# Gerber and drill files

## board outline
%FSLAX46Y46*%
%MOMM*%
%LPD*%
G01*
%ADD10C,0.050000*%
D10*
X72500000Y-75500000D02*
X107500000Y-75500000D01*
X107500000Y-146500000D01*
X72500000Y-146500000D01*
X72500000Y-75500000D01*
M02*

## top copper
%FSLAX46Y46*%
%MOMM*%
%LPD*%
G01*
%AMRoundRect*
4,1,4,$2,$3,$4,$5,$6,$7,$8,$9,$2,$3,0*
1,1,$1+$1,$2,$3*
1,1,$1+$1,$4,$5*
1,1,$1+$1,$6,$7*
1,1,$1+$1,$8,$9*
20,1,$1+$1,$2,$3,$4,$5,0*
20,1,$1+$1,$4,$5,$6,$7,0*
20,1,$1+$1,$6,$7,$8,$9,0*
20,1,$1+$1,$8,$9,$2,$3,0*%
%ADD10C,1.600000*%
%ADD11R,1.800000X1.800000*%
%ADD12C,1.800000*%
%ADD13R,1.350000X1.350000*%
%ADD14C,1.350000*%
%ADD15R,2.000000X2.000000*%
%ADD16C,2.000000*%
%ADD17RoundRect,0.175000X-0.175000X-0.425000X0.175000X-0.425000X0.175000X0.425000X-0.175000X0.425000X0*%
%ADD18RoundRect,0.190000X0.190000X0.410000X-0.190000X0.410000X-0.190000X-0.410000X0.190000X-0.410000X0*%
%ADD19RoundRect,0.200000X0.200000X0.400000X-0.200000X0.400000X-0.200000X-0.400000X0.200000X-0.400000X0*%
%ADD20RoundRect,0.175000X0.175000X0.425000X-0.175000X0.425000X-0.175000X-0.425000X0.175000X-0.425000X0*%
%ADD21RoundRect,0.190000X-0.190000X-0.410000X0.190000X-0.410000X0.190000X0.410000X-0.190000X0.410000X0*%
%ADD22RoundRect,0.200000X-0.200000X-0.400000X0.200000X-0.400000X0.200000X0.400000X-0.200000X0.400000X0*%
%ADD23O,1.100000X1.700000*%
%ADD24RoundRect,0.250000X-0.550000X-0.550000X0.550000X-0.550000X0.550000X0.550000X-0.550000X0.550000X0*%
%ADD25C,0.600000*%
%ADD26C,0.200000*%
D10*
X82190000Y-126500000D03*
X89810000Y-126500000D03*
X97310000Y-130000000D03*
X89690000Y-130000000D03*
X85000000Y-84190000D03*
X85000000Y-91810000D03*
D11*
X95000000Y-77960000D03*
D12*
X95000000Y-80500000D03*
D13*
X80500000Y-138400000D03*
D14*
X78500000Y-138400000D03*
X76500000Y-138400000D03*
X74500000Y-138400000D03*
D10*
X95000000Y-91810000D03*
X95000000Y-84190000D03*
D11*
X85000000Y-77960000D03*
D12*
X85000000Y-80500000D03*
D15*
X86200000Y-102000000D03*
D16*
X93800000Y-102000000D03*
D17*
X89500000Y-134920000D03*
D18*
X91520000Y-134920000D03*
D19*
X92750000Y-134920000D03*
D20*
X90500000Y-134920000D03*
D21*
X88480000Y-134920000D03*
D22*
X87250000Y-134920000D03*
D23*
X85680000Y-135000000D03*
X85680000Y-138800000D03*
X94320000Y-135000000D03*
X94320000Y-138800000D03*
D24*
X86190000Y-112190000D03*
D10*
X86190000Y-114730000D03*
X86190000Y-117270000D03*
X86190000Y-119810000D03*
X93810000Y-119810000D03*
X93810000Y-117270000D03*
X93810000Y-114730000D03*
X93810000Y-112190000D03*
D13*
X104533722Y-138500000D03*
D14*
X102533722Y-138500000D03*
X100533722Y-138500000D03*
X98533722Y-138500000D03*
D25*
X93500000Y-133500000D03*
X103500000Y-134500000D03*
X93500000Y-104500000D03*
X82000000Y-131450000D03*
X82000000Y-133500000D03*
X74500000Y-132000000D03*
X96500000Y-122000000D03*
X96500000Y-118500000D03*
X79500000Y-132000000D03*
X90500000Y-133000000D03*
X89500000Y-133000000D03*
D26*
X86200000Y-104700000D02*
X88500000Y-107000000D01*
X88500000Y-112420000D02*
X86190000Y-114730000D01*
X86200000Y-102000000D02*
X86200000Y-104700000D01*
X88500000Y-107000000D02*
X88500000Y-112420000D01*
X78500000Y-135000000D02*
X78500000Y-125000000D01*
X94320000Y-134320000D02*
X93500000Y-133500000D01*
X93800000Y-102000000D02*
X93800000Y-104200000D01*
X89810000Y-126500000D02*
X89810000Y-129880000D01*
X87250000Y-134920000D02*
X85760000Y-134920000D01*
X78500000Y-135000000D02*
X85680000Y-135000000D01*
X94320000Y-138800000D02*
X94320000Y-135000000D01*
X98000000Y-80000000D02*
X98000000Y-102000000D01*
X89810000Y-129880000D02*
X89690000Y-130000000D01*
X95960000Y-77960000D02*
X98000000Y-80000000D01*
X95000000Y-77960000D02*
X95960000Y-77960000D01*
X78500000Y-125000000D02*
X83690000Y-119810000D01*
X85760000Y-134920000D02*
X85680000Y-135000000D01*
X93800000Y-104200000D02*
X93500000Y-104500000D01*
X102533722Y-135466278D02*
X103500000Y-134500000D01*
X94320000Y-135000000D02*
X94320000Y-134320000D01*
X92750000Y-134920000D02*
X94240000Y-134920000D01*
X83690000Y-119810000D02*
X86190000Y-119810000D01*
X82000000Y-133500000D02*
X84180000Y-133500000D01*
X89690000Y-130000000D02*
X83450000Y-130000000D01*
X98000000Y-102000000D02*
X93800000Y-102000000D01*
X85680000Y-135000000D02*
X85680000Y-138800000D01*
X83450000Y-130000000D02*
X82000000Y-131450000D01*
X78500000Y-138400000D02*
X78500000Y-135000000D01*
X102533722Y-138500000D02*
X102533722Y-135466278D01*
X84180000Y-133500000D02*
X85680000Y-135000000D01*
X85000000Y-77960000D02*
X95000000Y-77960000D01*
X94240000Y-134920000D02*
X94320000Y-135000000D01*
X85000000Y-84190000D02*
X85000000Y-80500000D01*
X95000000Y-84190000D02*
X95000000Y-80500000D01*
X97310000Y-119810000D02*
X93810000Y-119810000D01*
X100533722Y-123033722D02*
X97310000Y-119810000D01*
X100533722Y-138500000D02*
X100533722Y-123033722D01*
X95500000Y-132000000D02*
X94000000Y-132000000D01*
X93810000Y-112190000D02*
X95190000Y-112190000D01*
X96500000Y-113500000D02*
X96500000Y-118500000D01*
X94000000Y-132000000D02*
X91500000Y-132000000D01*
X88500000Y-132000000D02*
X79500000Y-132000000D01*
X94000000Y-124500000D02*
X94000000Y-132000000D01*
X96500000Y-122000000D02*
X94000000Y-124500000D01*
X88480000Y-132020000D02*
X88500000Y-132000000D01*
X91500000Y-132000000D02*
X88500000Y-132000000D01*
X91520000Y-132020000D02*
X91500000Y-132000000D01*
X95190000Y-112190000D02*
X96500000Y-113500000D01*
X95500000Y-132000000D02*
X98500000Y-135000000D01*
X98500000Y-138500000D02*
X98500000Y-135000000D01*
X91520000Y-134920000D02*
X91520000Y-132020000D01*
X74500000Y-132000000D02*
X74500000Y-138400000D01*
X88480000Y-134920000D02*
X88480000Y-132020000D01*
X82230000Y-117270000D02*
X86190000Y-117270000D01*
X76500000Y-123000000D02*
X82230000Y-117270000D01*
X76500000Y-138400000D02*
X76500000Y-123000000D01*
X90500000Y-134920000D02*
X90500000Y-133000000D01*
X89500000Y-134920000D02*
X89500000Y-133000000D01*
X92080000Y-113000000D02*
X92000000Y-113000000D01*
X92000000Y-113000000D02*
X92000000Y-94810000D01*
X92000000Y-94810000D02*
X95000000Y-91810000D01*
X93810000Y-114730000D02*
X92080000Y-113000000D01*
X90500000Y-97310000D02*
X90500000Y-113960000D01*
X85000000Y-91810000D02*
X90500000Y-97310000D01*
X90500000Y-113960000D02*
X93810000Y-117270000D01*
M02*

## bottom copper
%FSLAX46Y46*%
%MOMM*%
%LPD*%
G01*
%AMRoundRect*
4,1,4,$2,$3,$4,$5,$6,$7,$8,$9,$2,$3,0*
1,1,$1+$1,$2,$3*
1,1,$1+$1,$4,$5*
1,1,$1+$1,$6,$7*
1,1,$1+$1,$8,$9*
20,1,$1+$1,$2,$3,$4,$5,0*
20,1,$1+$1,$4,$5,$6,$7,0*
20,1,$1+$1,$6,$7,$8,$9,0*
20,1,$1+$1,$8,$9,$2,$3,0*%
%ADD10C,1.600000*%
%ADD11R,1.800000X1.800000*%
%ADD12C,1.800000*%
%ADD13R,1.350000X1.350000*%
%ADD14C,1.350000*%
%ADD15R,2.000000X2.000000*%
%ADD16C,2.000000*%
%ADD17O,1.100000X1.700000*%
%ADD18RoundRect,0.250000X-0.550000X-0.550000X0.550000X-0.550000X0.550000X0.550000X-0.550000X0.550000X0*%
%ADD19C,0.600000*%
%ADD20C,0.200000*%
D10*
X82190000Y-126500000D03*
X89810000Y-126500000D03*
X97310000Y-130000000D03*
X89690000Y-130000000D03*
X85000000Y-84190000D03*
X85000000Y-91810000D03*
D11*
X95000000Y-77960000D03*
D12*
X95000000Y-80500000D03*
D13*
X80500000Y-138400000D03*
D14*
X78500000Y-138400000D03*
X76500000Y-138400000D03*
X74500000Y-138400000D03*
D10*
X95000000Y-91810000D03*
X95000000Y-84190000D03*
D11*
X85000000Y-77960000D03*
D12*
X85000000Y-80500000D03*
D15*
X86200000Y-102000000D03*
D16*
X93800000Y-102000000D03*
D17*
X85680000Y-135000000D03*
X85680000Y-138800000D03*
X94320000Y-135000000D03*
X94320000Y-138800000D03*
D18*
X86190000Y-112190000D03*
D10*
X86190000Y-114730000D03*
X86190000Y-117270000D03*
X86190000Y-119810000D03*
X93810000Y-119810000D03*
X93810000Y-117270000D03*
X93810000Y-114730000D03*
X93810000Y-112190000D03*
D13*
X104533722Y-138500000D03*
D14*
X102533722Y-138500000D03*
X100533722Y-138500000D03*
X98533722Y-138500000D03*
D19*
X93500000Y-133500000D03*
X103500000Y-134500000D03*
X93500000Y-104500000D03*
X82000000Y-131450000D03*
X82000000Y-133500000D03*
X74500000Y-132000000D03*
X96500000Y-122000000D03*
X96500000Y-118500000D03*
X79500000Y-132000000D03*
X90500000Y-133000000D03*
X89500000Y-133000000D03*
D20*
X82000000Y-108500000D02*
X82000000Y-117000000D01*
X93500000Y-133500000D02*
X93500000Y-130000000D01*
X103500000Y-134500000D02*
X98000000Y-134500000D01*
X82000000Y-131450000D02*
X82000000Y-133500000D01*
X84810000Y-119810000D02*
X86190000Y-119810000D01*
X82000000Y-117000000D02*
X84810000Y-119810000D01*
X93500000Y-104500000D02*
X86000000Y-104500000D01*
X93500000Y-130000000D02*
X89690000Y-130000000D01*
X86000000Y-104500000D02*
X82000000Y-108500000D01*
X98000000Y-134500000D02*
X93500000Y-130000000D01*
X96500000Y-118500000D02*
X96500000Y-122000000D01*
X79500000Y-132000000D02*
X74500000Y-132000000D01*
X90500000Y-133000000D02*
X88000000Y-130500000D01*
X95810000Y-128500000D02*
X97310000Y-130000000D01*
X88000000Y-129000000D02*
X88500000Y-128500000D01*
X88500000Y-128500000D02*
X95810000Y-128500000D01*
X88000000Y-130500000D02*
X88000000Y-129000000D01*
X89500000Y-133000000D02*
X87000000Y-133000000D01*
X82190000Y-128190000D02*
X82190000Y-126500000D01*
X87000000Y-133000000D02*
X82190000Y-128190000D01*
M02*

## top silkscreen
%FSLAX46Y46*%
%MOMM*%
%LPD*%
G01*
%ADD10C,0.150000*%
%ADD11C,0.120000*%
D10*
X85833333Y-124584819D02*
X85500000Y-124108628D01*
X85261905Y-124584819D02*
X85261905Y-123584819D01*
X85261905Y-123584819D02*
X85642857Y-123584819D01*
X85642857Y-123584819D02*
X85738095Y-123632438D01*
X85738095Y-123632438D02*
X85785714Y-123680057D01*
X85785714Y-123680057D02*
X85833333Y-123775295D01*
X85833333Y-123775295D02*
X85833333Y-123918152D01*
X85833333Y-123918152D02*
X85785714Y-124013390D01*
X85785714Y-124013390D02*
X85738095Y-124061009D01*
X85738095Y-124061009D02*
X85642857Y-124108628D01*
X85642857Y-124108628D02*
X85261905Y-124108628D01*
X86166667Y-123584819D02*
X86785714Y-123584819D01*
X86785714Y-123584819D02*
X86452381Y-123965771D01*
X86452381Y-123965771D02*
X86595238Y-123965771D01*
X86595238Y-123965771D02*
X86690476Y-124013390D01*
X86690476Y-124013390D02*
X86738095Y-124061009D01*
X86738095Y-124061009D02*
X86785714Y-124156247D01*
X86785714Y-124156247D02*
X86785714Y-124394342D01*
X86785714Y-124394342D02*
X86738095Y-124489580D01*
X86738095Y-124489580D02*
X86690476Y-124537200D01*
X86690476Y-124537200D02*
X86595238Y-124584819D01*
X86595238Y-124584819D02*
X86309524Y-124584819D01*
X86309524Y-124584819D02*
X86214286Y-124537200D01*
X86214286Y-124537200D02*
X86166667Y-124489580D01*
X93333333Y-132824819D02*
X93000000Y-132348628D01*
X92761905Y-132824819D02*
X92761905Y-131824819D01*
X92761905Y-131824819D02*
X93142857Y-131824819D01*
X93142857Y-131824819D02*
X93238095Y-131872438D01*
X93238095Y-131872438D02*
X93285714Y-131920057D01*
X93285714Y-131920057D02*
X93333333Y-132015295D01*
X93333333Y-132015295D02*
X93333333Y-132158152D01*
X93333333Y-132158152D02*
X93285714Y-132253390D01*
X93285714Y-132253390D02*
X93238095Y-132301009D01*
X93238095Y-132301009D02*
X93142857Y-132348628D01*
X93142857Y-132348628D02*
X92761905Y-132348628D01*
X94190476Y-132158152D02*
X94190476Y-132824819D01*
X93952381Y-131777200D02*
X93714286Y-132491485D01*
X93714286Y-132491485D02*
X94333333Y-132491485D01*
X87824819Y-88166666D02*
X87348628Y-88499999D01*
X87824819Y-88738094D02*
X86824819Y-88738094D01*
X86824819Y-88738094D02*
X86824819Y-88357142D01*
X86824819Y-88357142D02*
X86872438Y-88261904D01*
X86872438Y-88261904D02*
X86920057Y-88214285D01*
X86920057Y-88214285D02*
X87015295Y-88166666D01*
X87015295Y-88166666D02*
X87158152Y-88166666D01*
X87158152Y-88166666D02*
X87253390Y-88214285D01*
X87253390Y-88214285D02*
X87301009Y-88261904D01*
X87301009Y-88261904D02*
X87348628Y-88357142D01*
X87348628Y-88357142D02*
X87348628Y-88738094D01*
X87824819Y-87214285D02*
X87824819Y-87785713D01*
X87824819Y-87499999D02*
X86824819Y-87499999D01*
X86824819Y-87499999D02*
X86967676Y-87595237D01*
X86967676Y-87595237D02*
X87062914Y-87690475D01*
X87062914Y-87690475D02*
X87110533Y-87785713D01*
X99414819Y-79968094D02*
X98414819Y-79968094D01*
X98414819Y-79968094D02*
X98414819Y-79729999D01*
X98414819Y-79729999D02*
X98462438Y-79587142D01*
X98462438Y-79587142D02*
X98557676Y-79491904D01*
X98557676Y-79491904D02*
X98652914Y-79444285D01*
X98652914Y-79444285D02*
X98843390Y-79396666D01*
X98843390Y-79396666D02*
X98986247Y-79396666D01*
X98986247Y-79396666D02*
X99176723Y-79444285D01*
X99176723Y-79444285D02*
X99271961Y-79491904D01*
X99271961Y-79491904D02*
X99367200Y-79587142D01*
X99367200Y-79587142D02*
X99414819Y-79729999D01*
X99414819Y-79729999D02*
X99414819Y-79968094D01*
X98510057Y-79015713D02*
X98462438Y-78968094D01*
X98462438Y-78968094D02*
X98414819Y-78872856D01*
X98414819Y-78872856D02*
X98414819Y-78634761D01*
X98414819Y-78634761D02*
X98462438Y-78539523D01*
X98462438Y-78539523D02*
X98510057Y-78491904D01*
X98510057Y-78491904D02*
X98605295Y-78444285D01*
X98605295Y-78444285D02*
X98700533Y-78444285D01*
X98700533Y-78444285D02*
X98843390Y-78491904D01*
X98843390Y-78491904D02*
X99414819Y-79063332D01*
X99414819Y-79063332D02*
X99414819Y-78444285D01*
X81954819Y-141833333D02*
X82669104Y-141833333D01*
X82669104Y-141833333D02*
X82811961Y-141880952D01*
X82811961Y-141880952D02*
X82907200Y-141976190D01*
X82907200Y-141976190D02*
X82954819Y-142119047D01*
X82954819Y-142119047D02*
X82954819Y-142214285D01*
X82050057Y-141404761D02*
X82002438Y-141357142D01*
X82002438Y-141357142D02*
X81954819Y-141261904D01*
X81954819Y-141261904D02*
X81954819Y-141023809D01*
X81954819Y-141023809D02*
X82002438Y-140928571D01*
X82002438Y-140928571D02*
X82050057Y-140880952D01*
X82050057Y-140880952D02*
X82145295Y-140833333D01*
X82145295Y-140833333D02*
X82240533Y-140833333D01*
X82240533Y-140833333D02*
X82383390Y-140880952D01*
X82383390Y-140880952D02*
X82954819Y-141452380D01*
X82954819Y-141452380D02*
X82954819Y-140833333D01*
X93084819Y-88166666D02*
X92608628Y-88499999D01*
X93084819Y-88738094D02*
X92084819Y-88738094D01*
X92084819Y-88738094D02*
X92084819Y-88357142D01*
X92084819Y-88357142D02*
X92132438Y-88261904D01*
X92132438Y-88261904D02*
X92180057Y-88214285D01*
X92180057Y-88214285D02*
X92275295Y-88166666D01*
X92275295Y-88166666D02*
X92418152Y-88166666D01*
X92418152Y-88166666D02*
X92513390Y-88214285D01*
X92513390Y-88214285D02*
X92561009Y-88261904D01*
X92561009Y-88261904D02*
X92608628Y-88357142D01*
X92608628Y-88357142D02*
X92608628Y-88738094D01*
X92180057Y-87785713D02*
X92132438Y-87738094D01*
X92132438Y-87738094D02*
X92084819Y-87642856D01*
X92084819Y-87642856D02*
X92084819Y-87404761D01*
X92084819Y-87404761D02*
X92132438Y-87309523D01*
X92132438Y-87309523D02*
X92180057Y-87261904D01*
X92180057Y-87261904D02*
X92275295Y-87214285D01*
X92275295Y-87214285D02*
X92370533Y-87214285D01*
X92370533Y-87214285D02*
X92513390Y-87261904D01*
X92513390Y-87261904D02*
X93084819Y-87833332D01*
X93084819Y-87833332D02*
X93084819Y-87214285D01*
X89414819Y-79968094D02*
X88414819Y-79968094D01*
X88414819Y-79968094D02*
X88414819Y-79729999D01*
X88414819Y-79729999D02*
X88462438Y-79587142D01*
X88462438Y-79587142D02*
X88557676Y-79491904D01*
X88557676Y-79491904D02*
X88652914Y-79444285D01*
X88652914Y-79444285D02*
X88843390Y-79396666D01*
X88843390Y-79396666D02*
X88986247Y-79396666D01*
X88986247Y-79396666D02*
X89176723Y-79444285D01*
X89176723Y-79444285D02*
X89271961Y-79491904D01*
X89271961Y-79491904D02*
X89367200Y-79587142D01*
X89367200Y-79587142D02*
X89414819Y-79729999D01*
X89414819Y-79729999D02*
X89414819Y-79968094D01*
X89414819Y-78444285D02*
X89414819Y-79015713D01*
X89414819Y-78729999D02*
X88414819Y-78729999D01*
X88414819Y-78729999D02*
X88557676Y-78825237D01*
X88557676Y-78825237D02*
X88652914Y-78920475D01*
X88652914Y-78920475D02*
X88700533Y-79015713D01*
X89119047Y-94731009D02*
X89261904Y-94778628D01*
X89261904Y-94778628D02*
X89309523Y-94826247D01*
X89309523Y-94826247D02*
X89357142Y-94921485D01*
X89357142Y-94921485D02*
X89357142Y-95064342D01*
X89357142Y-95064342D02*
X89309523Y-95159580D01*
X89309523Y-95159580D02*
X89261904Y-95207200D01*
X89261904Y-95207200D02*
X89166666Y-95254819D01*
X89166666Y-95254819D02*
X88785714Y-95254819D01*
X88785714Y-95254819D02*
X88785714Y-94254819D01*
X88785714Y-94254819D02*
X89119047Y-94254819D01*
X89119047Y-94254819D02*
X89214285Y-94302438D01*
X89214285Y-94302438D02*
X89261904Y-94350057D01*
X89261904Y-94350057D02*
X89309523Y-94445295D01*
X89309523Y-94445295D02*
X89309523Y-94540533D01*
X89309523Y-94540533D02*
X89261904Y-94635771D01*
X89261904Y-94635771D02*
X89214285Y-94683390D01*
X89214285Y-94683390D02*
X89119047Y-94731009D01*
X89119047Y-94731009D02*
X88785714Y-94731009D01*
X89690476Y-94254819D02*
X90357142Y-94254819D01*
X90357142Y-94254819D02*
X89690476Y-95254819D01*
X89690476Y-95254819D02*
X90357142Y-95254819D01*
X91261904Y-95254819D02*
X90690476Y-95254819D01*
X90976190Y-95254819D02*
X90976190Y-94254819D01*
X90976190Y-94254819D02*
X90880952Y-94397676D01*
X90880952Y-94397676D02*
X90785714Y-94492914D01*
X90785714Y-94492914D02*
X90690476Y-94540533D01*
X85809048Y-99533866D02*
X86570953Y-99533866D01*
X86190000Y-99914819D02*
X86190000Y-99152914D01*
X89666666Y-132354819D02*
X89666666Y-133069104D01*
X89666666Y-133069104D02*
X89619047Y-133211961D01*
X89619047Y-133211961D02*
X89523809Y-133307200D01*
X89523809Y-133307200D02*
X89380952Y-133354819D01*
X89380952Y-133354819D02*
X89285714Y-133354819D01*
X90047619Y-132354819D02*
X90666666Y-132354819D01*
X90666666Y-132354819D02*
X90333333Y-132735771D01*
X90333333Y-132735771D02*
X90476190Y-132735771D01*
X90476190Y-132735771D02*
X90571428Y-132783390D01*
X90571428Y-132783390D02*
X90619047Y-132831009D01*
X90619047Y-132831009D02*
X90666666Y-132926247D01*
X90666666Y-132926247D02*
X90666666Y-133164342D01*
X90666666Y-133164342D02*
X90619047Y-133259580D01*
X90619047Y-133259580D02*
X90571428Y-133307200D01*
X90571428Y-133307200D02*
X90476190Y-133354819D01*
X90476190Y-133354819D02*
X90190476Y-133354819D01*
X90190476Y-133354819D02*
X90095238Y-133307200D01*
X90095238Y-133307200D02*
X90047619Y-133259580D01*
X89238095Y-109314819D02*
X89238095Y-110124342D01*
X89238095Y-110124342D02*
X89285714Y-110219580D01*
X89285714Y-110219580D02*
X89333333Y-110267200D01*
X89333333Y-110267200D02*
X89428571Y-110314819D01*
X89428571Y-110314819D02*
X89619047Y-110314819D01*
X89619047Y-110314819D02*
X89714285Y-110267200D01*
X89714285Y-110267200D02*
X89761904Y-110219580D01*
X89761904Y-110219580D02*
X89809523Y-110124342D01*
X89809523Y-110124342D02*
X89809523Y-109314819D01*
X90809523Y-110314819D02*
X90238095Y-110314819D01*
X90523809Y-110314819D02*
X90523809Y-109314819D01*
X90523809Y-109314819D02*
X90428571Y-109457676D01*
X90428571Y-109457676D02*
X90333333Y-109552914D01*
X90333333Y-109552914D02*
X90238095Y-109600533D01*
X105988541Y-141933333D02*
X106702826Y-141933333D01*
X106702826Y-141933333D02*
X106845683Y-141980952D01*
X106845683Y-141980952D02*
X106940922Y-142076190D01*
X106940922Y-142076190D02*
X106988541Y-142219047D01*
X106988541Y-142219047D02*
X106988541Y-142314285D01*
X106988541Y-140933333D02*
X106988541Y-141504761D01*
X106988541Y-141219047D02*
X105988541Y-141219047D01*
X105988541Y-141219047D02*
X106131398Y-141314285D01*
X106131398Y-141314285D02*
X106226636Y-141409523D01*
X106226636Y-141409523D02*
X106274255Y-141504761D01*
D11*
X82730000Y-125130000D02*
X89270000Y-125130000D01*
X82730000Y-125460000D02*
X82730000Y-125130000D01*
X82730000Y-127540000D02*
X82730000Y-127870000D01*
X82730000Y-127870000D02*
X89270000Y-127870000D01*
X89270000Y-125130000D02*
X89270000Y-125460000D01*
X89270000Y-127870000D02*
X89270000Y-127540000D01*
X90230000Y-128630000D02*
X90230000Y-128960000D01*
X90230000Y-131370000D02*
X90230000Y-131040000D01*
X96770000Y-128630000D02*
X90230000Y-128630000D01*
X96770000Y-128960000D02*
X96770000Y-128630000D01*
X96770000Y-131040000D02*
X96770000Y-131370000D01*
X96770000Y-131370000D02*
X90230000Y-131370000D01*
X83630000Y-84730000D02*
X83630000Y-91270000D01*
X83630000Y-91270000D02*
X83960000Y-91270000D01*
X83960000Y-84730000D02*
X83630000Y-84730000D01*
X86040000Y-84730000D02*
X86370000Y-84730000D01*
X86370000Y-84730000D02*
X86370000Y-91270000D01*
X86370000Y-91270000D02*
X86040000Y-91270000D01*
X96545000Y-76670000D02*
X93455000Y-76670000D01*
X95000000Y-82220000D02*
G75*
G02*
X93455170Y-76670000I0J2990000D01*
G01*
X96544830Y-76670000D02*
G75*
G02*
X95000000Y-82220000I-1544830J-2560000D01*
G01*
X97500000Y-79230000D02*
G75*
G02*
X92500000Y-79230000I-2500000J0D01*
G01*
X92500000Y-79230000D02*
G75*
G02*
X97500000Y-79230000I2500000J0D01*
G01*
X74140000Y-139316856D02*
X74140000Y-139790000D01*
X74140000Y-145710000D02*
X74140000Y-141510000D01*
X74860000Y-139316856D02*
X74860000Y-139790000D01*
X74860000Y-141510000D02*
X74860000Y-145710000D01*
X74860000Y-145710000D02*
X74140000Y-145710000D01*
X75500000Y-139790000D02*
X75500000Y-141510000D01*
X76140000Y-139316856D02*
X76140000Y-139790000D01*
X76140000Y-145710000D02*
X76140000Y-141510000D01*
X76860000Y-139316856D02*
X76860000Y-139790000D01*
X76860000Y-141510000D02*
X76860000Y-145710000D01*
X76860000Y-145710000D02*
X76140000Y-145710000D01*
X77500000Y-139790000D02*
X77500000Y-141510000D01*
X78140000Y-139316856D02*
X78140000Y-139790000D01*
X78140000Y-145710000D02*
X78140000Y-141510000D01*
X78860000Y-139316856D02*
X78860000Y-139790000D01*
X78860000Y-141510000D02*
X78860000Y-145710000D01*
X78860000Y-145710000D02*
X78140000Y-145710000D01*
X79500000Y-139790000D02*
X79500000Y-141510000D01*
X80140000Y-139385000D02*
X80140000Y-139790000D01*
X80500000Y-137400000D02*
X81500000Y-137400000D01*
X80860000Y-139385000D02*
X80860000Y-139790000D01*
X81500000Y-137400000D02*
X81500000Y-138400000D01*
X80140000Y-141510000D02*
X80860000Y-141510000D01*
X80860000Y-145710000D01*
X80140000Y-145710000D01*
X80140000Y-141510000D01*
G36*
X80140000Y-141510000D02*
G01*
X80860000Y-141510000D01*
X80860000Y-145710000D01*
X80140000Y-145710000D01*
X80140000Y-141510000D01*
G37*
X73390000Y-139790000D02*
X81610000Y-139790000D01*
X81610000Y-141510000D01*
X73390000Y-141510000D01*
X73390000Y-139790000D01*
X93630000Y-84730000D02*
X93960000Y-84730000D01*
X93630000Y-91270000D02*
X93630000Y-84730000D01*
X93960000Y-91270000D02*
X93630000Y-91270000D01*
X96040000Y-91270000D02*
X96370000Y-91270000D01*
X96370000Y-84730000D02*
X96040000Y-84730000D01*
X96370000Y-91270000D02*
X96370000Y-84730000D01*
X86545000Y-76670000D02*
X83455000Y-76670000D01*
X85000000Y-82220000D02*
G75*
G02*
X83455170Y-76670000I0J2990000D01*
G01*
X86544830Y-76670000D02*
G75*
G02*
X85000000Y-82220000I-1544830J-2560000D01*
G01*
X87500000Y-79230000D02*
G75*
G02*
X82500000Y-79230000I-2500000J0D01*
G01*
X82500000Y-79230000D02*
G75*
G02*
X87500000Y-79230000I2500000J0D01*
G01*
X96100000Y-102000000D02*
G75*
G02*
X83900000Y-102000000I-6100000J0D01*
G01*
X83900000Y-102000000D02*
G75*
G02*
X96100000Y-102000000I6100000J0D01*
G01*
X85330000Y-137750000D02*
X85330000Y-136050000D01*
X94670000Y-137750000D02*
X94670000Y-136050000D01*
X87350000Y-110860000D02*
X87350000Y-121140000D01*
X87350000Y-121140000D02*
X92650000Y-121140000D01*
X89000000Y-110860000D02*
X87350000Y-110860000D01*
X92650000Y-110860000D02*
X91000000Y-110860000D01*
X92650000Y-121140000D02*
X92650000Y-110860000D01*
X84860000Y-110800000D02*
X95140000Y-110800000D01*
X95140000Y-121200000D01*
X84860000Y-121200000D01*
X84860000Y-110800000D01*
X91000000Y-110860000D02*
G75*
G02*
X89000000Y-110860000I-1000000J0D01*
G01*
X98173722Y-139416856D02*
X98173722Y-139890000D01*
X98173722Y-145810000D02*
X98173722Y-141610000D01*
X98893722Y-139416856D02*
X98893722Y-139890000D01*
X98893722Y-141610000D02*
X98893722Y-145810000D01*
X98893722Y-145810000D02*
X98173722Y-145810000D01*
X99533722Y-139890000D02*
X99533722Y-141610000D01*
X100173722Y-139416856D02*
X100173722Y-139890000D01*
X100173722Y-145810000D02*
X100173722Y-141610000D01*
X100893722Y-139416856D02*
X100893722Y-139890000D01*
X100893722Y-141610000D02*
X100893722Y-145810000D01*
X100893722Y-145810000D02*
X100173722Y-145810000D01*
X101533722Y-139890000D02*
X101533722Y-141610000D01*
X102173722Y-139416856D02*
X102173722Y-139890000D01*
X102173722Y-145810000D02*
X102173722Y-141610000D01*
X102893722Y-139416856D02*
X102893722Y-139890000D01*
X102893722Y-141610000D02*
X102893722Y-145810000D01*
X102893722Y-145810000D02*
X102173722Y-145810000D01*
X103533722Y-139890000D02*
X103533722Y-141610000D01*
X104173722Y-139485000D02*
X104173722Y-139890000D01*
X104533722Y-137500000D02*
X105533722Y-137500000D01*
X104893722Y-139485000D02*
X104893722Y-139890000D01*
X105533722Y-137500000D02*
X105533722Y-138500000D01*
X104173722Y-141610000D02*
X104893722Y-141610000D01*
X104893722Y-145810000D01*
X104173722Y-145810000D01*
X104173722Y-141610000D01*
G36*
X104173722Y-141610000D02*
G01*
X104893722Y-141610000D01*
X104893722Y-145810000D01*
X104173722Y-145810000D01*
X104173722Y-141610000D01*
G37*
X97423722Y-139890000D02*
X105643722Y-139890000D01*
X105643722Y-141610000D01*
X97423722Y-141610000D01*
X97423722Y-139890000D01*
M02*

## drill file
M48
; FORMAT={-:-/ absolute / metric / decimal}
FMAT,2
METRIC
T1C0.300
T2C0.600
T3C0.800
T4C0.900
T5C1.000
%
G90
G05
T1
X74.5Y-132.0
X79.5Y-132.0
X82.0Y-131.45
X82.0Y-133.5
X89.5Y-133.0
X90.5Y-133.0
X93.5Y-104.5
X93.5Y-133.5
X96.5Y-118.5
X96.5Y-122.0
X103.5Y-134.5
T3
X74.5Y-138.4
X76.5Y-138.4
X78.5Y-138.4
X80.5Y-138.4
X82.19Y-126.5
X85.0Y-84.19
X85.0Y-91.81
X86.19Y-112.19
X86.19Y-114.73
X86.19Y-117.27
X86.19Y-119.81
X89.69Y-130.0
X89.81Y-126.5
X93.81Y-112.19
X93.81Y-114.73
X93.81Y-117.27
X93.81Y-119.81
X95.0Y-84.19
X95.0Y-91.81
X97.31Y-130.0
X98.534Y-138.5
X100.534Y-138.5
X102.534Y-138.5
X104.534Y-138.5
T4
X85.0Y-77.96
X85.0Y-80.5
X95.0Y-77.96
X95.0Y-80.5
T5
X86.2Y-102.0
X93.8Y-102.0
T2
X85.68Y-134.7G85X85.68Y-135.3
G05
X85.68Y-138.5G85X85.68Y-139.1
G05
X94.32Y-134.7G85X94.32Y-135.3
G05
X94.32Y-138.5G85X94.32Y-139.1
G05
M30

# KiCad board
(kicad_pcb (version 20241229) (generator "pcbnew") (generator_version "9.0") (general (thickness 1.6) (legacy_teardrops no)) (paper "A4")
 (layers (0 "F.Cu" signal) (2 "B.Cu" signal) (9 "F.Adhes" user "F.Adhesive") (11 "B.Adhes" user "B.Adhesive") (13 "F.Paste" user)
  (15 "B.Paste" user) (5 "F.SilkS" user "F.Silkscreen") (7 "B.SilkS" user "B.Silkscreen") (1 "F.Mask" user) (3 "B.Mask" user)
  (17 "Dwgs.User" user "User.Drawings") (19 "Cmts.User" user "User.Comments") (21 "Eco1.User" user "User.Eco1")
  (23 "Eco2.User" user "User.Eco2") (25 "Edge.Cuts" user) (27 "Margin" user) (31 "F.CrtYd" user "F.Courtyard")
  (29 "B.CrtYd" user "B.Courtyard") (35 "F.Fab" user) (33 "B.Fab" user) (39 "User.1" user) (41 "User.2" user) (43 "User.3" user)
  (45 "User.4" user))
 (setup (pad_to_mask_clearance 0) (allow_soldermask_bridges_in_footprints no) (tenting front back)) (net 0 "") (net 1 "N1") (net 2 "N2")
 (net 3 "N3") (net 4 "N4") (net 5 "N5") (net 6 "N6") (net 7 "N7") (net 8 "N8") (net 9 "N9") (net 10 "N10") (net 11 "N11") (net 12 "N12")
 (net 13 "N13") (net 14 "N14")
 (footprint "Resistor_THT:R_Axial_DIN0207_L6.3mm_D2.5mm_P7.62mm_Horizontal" (layer "F.Cu") (at 82.19 126.5)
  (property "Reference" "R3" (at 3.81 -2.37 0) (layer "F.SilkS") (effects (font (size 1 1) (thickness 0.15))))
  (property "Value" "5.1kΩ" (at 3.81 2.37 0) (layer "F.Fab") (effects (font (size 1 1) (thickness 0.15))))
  (fp_line (start 0.54 -1.37) (end 7.08 -1.37) (stroke (width 0.12) (type solid)) (layer "F.SilkS"))
  (fp_line (start 0.54 -1.04) (end 0.54 -1.37) (stroke (width 0.12) (type solid)) (layer "F.SilkS"))
  (fp_line (start 0.54 1.04) (end 0.54 1.37) (stroke (width 0.12) (type solid)) (layer "F.SilkS"))
  (fp_line (start 0.54 1.37) (end 7.08 1.37) (stroke (width 0.12) (type solid)) (layer "F.SilkS"))
  (fp_line (start 7.08 -1.37) (end 7.08 -1.04) (stroke (width 0.12) (type solid)) (layer "F.SilkS"))
  (fp_line (start 7.08 1.37) (end 7.08 1.04) (stroke (width 0.12) (type solid)) (layer "F.SilkS"))
  (pad "1" thru_hole circle (at 0 0) (size 1.6 1.6) (drill 0.8) (layers "*.Cu" "*.Mask") (remove_unused_layers no) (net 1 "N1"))
  (pad "2" thru_hole circle (at 7.62 0) (size 1.6 1.6) (drill 0.8) (layers "*.Cu" "*.Mask") (remove_unused_layers no) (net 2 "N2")))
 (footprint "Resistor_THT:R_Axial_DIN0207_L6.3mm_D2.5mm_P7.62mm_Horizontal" (layer "F.Cu") (at 97.31 130 180)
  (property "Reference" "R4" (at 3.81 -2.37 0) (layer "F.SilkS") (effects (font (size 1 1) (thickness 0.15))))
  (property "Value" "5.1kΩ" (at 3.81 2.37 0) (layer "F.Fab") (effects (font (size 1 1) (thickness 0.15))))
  (fp_line (start 7.08 1.37) (end 7.08 1.04) (stroke (width 0.12) (type solid)) (layer "F.SilkS"))
  (fp_line (start 7.08 -1.37) (end 7.08 -1.04) (stroke (width 0.12) (type solid)) (layer "F.SilkS"))
  (fp_line (start 0.54 1.37) (end 7.08 1.37) (stroke (width 0.12) (type solid)) (layer "F.SilkS"))
  (fp_line (start 0.54 1.04) (end 0.54 1.37) (stroke (width 0.12) (type solid)) (layer "F.SilkS"))
  (fp_line (start 0.54 -1.04) (end 0.54 -1.37) (stroke (width 0.12) (type solid)) (layer "F.SilkS"))
  (fp_line (start 0.54 -1.37) (end 7.08 -1.37) (stroke (width 0.12) (type solid)) (layer "F.SilkS"))
  (pad "1" thru_hole circle (at 0 0 180) (size 1.6 1.6) (drill 0.8) (layers "*.Cu" "*.Mask") (remove_unused_layers no) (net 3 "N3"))
  (pad "2" thru_hole circle (at 7.62 0 180) (size 1.6 1.6) (drill 0.8) (layers "*.Cu" "*.Mask") (remove_unused_layers no) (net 2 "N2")))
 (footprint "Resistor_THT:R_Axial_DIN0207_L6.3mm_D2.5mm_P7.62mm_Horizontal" (layer "F.Cu") (at 85 84.19 -90)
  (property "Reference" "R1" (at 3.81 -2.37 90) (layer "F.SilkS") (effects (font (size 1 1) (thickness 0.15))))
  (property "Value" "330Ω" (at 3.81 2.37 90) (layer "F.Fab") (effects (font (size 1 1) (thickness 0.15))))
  (fp_line (start 0.54 1.37) (end 7.08 1.37) (stroke (width 0.12) (type solid)) (layer "F.SilkS"))
  (fp_line (start 7.08 1.37) (end 7.08 1.04) (stroke (width 0.12) (type solid)) (layer "F.SilkS"))
  (fp_line (start 0.54 1.04) (end 0.54 1.37) (stroke (width 0.12) (type solid)) (layer "F.SilkS"))
  (fp_line (start 0.54 -1.04) (end 0.54 -1.37) (stroke (width 0.12) (type solid)) (layer "F.SilkS"))
  (fp_line (start 0.54 -1.37) (end 7.08 -1.37) (stroke (width 0.12) (type solid)) (layer "F.SilkS"))
  (fp_line (start 7.08 -1.37) (end 7.08 -1.04) (stroke (width 0.12) (type solid)) (layer "F.SilkS"))
  (pad "1" thru_hole circle (at 0 0 270) (size 1.6 1.6) (drill 0.8) (layers "*.Cu" "*.Mask") (remove_unused_layers no) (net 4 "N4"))
  (pad "2" thru_hole circle (at 7.62 0 270) (size 1.6 1.6) (drill 0.8) (layers "*.Cu" "*.Mask") (remove_unused_layers no) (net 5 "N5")))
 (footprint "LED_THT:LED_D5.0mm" (layer "F.Cu") (at 95 77.96 -90)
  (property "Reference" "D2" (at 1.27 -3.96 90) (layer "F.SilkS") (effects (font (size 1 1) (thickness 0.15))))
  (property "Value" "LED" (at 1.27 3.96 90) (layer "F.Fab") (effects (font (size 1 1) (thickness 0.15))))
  (fp_line (start -1.29 -1.545) (end -1.29 1.545) (stroke (width 0.12) (type solid)) (layer "F.SilkS"))
  (fp_arc (start 4.26 0) (mid 2.071779 2.880495) (end -1.29 1.54483) (stroke (width 0.12) (type solid)) (layer "F.SilkS"))
  (fp_arc (start -1.29 -1.54483) (mid 2.071779 -2.880495) (end 4.26 0) (stroke (width 0.12) (type solid)) (layer "F.SilkS"))
  (fp_circle (center 1.27 0) (end 3.77 0) (stroke (width 0.12) (type solid)) (fill no) (layer "F.SilkS"))
  (pad "1" thru_hole rect (at 0 0 270) (size 1.8 1.8) (drill 0.9) (layers "*.Cu" "*.Mask") (remove_unused_layers no) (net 2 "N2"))
  (pad "2" thru_hole circle (at 2.54 0 270) (size 1.8 1.8) (drill 0.9) (layers "*.Cu" "*.Mask") (remove_unused_layers no) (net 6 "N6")))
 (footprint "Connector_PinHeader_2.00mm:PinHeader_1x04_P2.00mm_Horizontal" (layer "F.Cu") (at 80.5 138.4 -90)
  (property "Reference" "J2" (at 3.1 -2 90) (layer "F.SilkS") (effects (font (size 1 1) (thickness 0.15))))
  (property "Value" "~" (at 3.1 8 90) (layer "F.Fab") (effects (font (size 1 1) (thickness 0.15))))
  (fp_line (start 0.916856 6.36) (end 1.39 6.36) (stroke (width 0.12) (type solid)) (layer "F.SilkS"))
  (fp_line (start 7.31 6.36) (end 3.11 6.36) (stroke (width 0.12) (type solid)) (layer "F.SilkS"))
  (fp_line (start 0.916856 5.64) (end 1.39 5.64) (stroke (width 0.12) (type solid)) (layer "F.SilkS"))
  (fp_line (start 3.11 5.64) (end 7.31 5.64) (stroke (width 0.12) (type solid)) (layer "F.SilkS"))
  (fp_line (start 7.31 5.64) (end 7.31 6.36) (stroke (width 0.12) (type solid)) (layer "F.SilkS"))
  (fp_line (start 1.39 5) (end 3.11 5) (stroke (width 0.12) (type solid)) (layer "F.SilkS"))
  (fp_line (start 0.916856 4.36) (end 1.39 4.36) (stroke (width 0.12) (type solid)) (layer "F.SilkS"))
  (fp_line (start 7.31 4.36) (end 3.11 4.36) (stroke (width 0.12) (type solid)) (layer "F.SilkS"))
  (fp_line (start 0.916856 3.64) (end 1.39 3.64) (stroke (width 0.12) (type solid)) (layer "F.SilkS"))
  (fp_line (start 3.11 3.64) (end 7.31 3.64) (stroke (width 0.12) (type solid)) (layer "F.SilkS"))
  (fp_line (start 7.31 3.64) (end 7.31 4.36) (stroke (width 0.12) (type solid)) (layer "F.SilkS"))
  (fp_line (start 1.39 3) (end 3.11 3) (stroke (width 0.12) (type solid)) (layer "F.SilkS"))
  (fp_line (start 0.916856 2.36) (end 1.39 2.36) (stroke (width 0.12) (type solid)) (layer "F.SilkS"))
  (fp_line (start 7.31 2.36) (end 3.11 2.36) (stroke (width 0.12) (type solid)) (layer "F.SilkS"))
  (fp_line (start 0.916856 1.64) (end 1.39 1.64) (stroke (width 0.12) (type solid)) (layer "F.SilkS"))
  (fp_line (start 3.11 1.64) (end 7.31 1.64) (stroke (width 0.12) (type solid)) (layer "F.SilkS"))
  (fp_line (start 7.31 1.64) (end 7.31 2.36) (stroke (width 0.12) (type solid)) (layer "F.SilkS"))
  (fp_line (start 1.39 1) (end 3.11 1) (stroke (width 0.12) (type solid)) (layer "F.SilkS"))
  (fp_line (start 0.985 0.36) (end 1.39 0.36) (stroke (width 0.12) (type solid)) (layer "F.SilkS"))
  (fp_line (start -1 0) (end -1 -1) (stroke (width 0.12) (type solid)) (layer "F.SilkS"))
  (fp_line (start 0.985 -0.36) (end 1.39 -0.36) (stroke (width 0.12) (type solid)) (layer "F.SilkS"))
  (fp_line (start -1 -1) (end 0 -1) (stroke (width 0.12) (type solid)) (layer "F.SilkS"))
  (fp_rect (start 3.11 -0.36) (end 7.31 0.36) (stroke (width 0.12) (type solid)) (fill yes) (layer "F.SilkS"))
  (fp_rect (start 1.39 -1.11) (end 3.11 7.11) (stroke (width 0.12) (type solid)) (fill no) (layer "F.SilkS"))
  (pad "1" thru_hole rect (at 0 0 270) (size 1.35 1.35) (drill 0.8) (layers "*.Cu" "*.Mask") (remove_unused_layers no) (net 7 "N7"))
  (pad "2" thru_hole circle (at 0 2 270) (size 1.35 1.35) (drill 0.8) (layers "*.Cu" "*.Mask") (remove_unused_layers no) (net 2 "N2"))
  (pad "3" thru_hole circle (at 0 4 270) (size 1.35 1.35) (drill 0.8) (layers "*.Cu" "*.Mask") (remove_unused_layers no) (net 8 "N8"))
  (pad "4" thru_hole circle (at 0 6 270) (size 1.35 1.35) (drill 0.8) (layers "*.Cu" "*.Mask") (remove_unused_layers no) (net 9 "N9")))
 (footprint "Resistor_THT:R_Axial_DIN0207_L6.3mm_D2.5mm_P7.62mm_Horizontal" (layer "F.Cu") (at 95 91.81 90)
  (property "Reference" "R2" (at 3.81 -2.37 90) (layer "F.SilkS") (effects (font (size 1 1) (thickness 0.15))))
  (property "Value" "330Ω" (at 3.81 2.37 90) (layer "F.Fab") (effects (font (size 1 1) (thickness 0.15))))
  (fp_line (start 7.08 -1.37) (end 7.08 -1.04) (stroke (width 0.12) (type solid)) (layer "F.SilkS"))
  (fp_line (start 0.54 -1.37) (end 7.08 -1.37) (stroke (width 0.12) (type solid)) (layer "F.SilkS"))
  (fp_line (start 0.54 -1.04) (end 0.54 -1.37) (stroke (width 0.12) (type solid)) (layer "F.SilkS"))
  (fp_line (start 0.54 1.04) (end 0.54 1.37) (stroke (width 0.12) (type solid)) (layer "F.SilkS"))
  (fp_line (start 7.08 1.37) (end 7.08 1.04) (stroke (width 0.12) (type solid)) (layer "F.SilkS"))
  (fp_line (start 0.54 1.37) (end 7.08 1.37) (stroke (width 0.12) (type solid)) (layer "F.SilkS"))
  (pad "1" thru_hole circle (at 0 0 90) (size 1.6 1.6) (drill 0.8) (layers "*.Cu" "*.Mask") (remove_unused_layers no) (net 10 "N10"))
  (pad "2" thru_hole circle (at 7.62 0 90) (size 1.6 1.6) (drill 0.8) (layers "*.Cu" "*.Mask") (remove_unused_layers no) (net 6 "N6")))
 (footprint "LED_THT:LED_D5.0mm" (layer "F.Cu") (at 85 77.96 -90)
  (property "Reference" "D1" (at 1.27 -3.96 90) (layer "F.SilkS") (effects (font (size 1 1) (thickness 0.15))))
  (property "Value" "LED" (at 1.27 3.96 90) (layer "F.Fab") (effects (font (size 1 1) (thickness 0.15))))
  (fp_line (start -1.29 -1.545) (end -1.29 1.545) (stroke (width 0.12) (type solid)) (layer "F.SilkS"))
  (fp_arc (start 4.26 0) (mid 2.071779 2.880495) (end -1.29 1.54483) (stroke (width 0.12) (type solid)) (layer "F.SilkS"))
  (fp_arc (start -1.29 -1.54483) (mid 2.071779 -2.880495) (end 4.26 0) (stroke (width 0.12) (type solid)) (layer "F.SilkS"))
  (fp_circle (center 1.27 0) (end 3.77 0) (stroke (width 0.12) (type solid)) (fill no) (layer "F.SilkS"))
  (pad "1" thru_hole rect (at 0 0 270) (size 1.8 1.8) (drill 0.9) (layers "*.Cu" "*.Mask") (remove_unused_layers no) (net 2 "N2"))
  (pad "2" thru_hole circle (at 2.54 0 270) (size 1.8 1.8) (drill 0.9) (layers "*.Cu" "*.Mask") (remove_unused_layers no) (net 4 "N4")))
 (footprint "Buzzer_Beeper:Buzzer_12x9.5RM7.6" (layer "F.Cu") (at 86.2 102)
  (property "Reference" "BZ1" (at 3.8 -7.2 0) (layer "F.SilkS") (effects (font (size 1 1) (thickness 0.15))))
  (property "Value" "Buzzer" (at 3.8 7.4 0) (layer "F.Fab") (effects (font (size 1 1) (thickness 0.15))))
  (fp_circle (center 3.8 0) (end 9.9 0) (stroke (width 0.12) (type solid)) (fill no) (layer "F.SilkS"))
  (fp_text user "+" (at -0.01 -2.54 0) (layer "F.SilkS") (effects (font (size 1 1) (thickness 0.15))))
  (pad "1" thru_hole rect (at 0 0) (size 2 2) (drill 1) (layers "*.Cu" "*.Mask") (remove_unused_layers no) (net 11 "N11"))
  (pad "2" thru_hole circle (at 7.6 0) (size 2 2) (drill 1) (layers "*.Cu" "*.Mask") (remove_unused_layers no) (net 2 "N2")))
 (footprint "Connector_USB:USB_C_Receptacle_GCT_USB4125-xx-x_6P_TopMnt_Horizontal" (layer "F.Cu") (at 90 138)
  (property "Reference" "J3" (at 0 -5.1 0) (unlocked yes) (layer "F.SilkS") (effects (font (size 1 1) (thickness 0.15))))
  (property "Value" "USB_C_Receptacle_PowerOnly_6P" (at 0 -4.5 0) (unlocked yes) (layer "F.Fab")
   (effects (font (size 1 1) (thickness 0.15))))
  (fp_line (start -4.67 -0.25) (end -4.67 -1.95) (stroke (width 0.12) (type solid)) (layer "F.SilkS"))
  (fp_line (start 4.67 -0.25) (end 4.67 -1.95) (stroke (width 0.12) (type solid)) (layer "F.SilkS"))
  (pad "A5" smd roundrect (at -0.5 -3.08) (size 0.7 1.2) (layers "F.Cu" "F.Mask" "F.Paste") (roundrect_rratio 0.25) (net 1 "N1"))
  (pad "A9" smd roundrect (at 1.52 -3.08 180) (size 0.76 1.2) (layers "F.Cu" "F.Mask" "F.Paste") (roundrect_rratio 0.25) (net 9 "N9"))
  (pad "A12" smd roundrect (at 2.75 -3.08 180) (size 0.8 1.2) (layers "F.Cu" "F.Mask" "F.Paste") (roundrect_rratio 0.25) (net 2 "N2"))
  (pad "B5" smd roundrect (at 0.5 -3.08 180) (size 0.7 1.2) (layers "F.Cu" "F.Mask" "F.Paste") (roundrect_rratio 0.25) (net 3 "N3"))
  (pad "B9" smd roundrect (at -1.52 -3.08) (size 0.76 1.2) (layers "F.Cu" "F.Mask" "F.Paste") (roundrect_rratio 0.25) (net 9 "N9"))
  (pad "B12" smd roundrect (at -2.75 -3.08) (size 0.8 1.2) (layers "F.Cu" "F.Mask" "F.Paste") (roundrect_rratio 0.25) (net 2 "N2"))
  (pad "S1" thru_hole oval (at -4.32 -3) (size 1.1 1.7) (drill oval 0.6 1.2) (layers "*.Cu" "*.Mask" "F.Paste") (remove_unused_layers no)
   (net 2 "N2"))
  (pad "S1" thru_hole oval (at -4.32 0.8) (size 1.1 1.7) (drill oval 0.6 1.2) (layers "*.Cu" "*.Mask" "F.Paste") (remove_unused_layers no)
   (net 2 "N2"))
  (pad "S1" thru_hole oval (at 4.32 -3) (size 1.1 1.7) (drill oval 0.6 1.2) (layers "*.Cu" "*.Mask" "F.Paste") (remove_unused_layers no)
   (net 2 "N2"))
  (pad "S1" thru_hole oval (at 4.32 0.8) (size 1.1 1.7) (drill oval 0.6 1.2) (layers "*.Cu" "*.Mask" "F.Paste") (remove_unused_layers no)
   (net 2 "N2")))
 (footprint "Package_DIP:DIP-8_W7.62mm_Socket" (layer "F.Cu") (at 86.19 112.19)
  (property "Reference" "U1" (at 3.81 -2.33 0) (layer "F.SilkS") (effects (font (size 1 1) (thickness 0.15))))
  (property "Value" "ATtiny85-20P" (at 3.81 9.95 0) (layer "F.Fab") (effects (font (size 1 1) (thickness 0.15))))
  (fp_line (start 1.16 -1.33) (end 1.16 8.95) (stroke (width 0.12) (type solid)) (layer "F.SilkS"))
  (fp_line (start 1.16 8.95) (end 6.46 8.95) (stroke (width 0.12) (type solid)) (layer "F.SilkS"))
  (fp_line (start 2.81 -1.33) (end 1.16 -1.33) (stroke (width 0.12) (type solid)) (layer "F.SilkS"))
  (fp_line (start 6.46 -1.33) (end 4.81 -1.33) (stroke (width 0.12) (type solid)) (layer "F.SilkS"))
  (fp_line (start 6.46 8.95) (end 6.46 -1.33) (stroke (width 0.12) (type solid)) (layer "F.SilkS"))
  (fp_rect (start -1.33 -1.39) (end 8.95 9.01) (stroke (width 0.12) (type solid)) (fill no) (layer "F.SilkS"))
  (fp_arc (start 4.81 -1.33) (mid 3.81 -0.33) (end 2.81 -1.33) (stroke (width 0.12) (type solid)) (layer "F.SilkS"))
  (pad "1" thru_hole roundrect (at 0 0) (size 1.6 1.6) (drill 0.8) (layers "*.Cu" "*.Mask") (remove_unused_layers no)
   (roundrect_rratio 0.15625) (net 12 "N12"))
  (pad "2" thru_hole circle (at 0 2.54) (size 1.6 1.6) (drill 0.8) (layers "*.Cu" "*.Mask") (remove_unused_layers no) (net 11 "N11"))
  (pad "3" thru_hole circle (at 0 5.08) (size 1.6 1.6) (drill 0.8) (layers "*.Cu" "*.Mask") (remove_unused_layers no) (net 8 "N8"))
  (pad "4" thru_hole circle (at 0 7.62) (size 1.6 1.6) (drill 0.8) (layers "*.Cu" "*.Mask") (remove_unused_layers no) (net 2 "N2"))
  (pad "5" thru_hole circle (at 7.62 7.62) (size 1.6 1.6) (drill 0.8) (layers "*.Cu" "*.Mask") (remove_unused_layers no) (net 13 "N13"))
  (pad "6" thru_hole circle (at 7.62 5.08) (size 1.6 1.6) (drill 0.8) (layers "*.Cu" "*.Mask") (remove_unused_layers no) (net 5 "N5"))
  (pad "7" thru_hole circle (at 7.62 2.54) (size 1.6 1.6) (drill 0.8) (layers "*.Cu" "*.Mask") (remove_unused_layers no) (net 10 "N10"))
  (pad "8" thru_hole circle (at 7.62 0) (size 1.6 1.6) (drill 0.8) (layers "*.Cu" "*.Mask") (remove_unused_layers no) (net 9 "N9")))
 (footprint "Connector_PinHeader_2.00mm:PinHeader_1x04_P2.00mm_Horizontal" (layer "F.Cu") (at 104.533722 138.5 -90)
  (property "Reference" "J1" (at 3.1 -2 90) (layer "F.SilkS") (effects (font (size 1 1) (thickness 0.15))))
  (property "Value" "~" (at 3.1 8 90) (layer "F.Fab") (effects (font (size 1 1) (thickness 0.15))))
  (fp_line (start 0.916856 6.36) (end 1.39 6.36) (stroke (width 0.12) (type solid)) (layer "F.SilkS"))
  (fp_line (start 7.31 6.36) (end 3.11 6.36) (stroke (width 0.12) (type solid)) (layer "F.SilkS"))
  (fp_line (start 0.916856 5.64) (end 1.39 5.64) (stroke (width 0.12) (type solid)) (layer "F.SilkS"))
  (fp_line (start 3.11 5.64) (end 7.31 5.64) (stroke (width 0.12) (type solid)) (layer "F.SilkS"))
  (fp_line (start 7.31 5.64) (end 7.31 6.36) (stroke (width 0.12) (type solid)) (layer "F.SilkS"))
  (fp_line (start 1.39 5) (end 3.11 5) (stroke (width 0.12) (type solid)) (layer "F.SilkS"))
  (fp_line (start 0.916856 4.36) (end 1.39 4.36) (stroke (width 0.12) (type solid)) (layer "F.SilkS"))
  (fp_line (start 7.31 4.36) (end 3.11 4.36) (stroke (width 0.12) (type solid)) (layer "F.SilkS"))
  (fp_line (start 0.916856 3.64) (end 1.39 3.64) (stroke (width 0.12) (type solid)) (layer "F.SilkS"))
  (fp_line (start 3.11 3.64) (end 7.31 3.64) (stroke (width 0.12) (type solid)) (layer "F.SilkS"))
  (fp_line (start 7.31 3.64) (end 7.31 4.36) (stroke (width 0.12) (type solid)) (layer "F.SilkS"))
  (fp_line (start 1.39 3) (end 3.11 3) (stroke (width 0.12) (type solid)) (layer "F.SilkS"))
  (fp_line (start 0.916856 2.36) (end 1.39 2.36) (stroke (width 0.12) (type solid)) (layer "F.SilkS"))
  (fp_line (start 7.31 2.36) (end 3.11 2.36) (stroke (width 0.12) (type solid)) (layer "F.SilkS"))
  (fp_line (start 0.916856 1.64) (end 1.39 1.64) (stroke (width 0.12) (type solid)) (layer "F.SilkS"))
  (fp_line (start 3.11 1.64) (end 7.31 1.64) (stroke (width 0.12) (type solid)) (layer "F.SilkS"))
  (fp_line (start 7.31 1.64) (end 7.31 2.36) (stroke (width 0.12) (type solid)) (layer "F.SilkS"))
  (fp_line (start 1.39 1) (end 3.11 1) (stroke (width 0.12) (type solid)) (layer "F.SilkS"))
  (fp_line (start 0.985 0.36) (end 1.39 0.36) (stroke (width 0.12) (type solid)) (layer "F.SilkS"))
  (fp_line (start -1 0) (end -1 -1) (stroke (width 0.12) (type solid)) (layer "F.SilkS"))
  (fp_line (start 0.985 -0.36) (end 1.39 -0.36) (stroke (width 0.12) (type solid)) (layer "F.SilkS"))
  (fp_line (start -1 -1) (end 0 -1) (stroke (width 0.12) (type solid)) (layer "F.SilkS"))
  (fp_rect (start 3.11 -0.36) (end 7.31 0.36) (stroke (width 0.12) (type solid)) (fill yes) (layer "F.SilkS"))
  (fp_rect (start 1.39 -1.11) (end 3.11 7.11) (stroke (width 0.12) (type solid)) (fill no) (layer "F.SilkS"))
  (pad "1" thru_hole rect (at 0 0 270) (size 1.35 1.35) (drill 0.8) (layers "*.Cu" "*.Mask") (remove_unused_layers no) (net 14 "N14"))
  (pad "2" thru_hole circle (at 0 2 270) (size 1.35 1.35) (drill 0.8) (layers "*.Cu" "*.Mask") (remove_unused_layers no) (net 2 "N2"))
  (pad "3" thru_hole circle (at 0 4 270) (size 1.35 1.35) (drill 0.8) (layers "*.Cu" "*.Mask") (remove_unused_layers no) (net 13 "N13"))
  (pad "4" thru_hole circle (at 0 6 270) (size 1.35 1.35) (drill 0.8) (layers "*.Cu" "*.Mask") (remove_unused_layers no) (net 9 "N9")))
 (gr_rect (start 72.5 75.5) (end 107.5 146.5) (stroke (width 0.05) (type default)) (fill no) (layer "Edge.Cuts"))
 (segment (start 86.2 104.7) (end 88.5 107) (width 0.2) (layer "F.Cu") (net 11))
 (segment (start 88.5 112.42) (end 86.19 114.73) (width 0.2) (layer "F.Cu") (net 11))
 (segment (start 86.2 102) (end 86.2 104.7) (width 0.2) (layer "F.Cu") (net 11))
 (segment (start 88.5 107) (end 88.5 112.42) (width 0.2) (layer "F.Cu") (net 11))
 (segment (start 78.5 135) (end 78.5 125) (width 0.2) (layer "F.Cu") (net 2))
 (segment (start 94.32 134.32) (end 93.5 133.5) (width 0.2) (layer "F.Cu") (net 2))
 (segment (start 93.8 102) (end 93.8 104.2) (width 0.2) (layer "F.Cu") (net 2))
 (segment (start 89.81 126.5) (end 89.81 129.88) (width 0.2) (layer "F.Cu") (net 2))
 (segment (start 87.25 134.92) (end 85.76 134.92) (width 0.2) (layer "F.Cu") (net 2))
 (segment (start 78.5 135) (end 85.68 135) (width 0.2) (layer "F.Cu") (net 2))
 (segment (start 94.32 138.8) (end 94.32 135) (width 0.2) (layer "F.Cu") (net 2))
 (segment (start 98 80) (end 98 102) (width 0.2) (layer "F.Cu") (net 2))
 (segment (start 89.81 129.88) (end 89.69 130) (width 0.2) (layer "F.Cu") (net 2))
 (segment (start 95.96 77.96) (end 98 80) (width 0.2) (layer "F.Cu") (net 2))
 (segment (start 95 77.96) (end 95.96 77.96) (width 0.2) (layer "F.Cu") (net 2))
 (segment (start 78.5 125) (end 83.69 119.81) (width 0.2) (layer "F.Cu") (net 2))
 (segment (start 85.76 134.92) (end 85.68 135) (width 0.2) (layer "F.Cu") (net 2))
 (segment (start 93.8 104.2) (end 93.5 104.5) (width 0.2) (layer "F.Cu") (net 2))
 (segment (start 102.533722 135.466278) (end 103.5 134.5) (width 0.2) (layer "F.Cu") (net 2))
 (segment (start 94.32 135) (end 94.32 134.32) (width 0.2) (layer "F.Cu") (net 2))
 (segment (start 92.75 134.92) (end 94.24 134.92) (width 0.2) (layer "F.Cu") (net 2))
 (segment (start 83.69 119.81) (end 86.19 119.81) (width 0.2) (layer "F.Cu") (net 2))
 (segment (start 82 133.5) (end 84.18 133.5) (width 0.2) (layer "F.Cu") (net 2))
 (segment (start 89.69 130) (end 83.45 130) (width 0.2) (layer "F.Cu") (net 2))
 (segment (start 98 102) (end 93.8 102) (width 0.2) (layer "F.Cu") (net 2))
 (segment (start 85.68 135) (end 85.68 138.8) (width 0.2) (layer "F.Cu") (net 2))
 (segment (start 83.45 130) (end 82 131.45) (width 0.2) (layer "F.Cu") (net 2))
 (segment (start 78.5 138.4) (end 78.5 135) (width 0.2) (layer "F.Cu") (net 2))
 (segment (start 102.533722 138.5) (end 102.533722 135.466278) (width 0.2) (layer "F.Cu") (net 2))
 (segment (start 84.18 133.5) (end 85.68 135) (width 0.2) (layer "F.Cu") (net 2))
 (segment (start 85 77.96) (end 95 77.96) (width 0.2) (layer "F.Cu") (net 2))
 (segment (start 94.24 134.92) (end 94.32 135) (width 0.2) (layer "F.Cu") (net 2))
 (via (at 93.5 133.5) (size 0.6) (drill 0.3) (layers "F.Cu" "B.Cu") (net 2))
 (via (at 103.5 134.5) (size 0.6) (drill 0.3) (layers "F.Cu" "B.Cu") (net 2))
 (via (at 93.5 104.5) (size 0.6) (drill 0.3) (layers "F.Cu" "B.Cu") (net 2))
 (via (at 82 131.45) (size 0.6) (drill 0.3) (layers "F.Cu" "B.Cu") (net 2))
 (via (at 82 133.5) (size 0.6) (drill 0.3) (layers "F.Cu" "B.Cu") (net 2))
 (segment (start 82 108.5) (end 82 117) (width 0.2) (layer "B.Cu") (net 2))
 (segment (start 93.5 133.5) (end 93.5 130) (width 0.2) (layer "B.Cu") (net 2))
 (segment (start 103.5 134.5) (end 98 134.5) (width 0.2) (layer "B.Cu") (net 2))
 (segment (start 82 131.45) (end 82 133.5) (width 0.2) (layer "B.Cu") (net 2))
 (segment (start 84.81 119.81) (end 86.19 119.81) (width 0.2) (layer "B.Cu") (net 2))
 (segment (start 82 117) (end 84.81 119.81) (width 0.2) (layer "B.Cu") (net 2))
 (segment (start 93.5 104.5) (end 86 104.5) (width 0.2) (layer "B.Cu") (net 2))
 (segment (start 93.5 130) (end 89.69 130) (width 0.2) (layer "B.Cu") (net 2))
 (segment (start 86 104.5) (end 82 108.5) (width 0.2) (layer "B.Cu") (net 2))
 (segment (start 98 134.5) (end 93.5 130) (width 0.2) (layer "B.Cu") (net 2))
 (segment (start 85 84.19) (end 85 80.5) (width 0.2) (layer "F.Cu") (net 4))
 (segment (start 95 84.19) (end 95 80.5) (width 0.2) (layer "F.Cu") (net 6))
 (segment (start 97.31 119.81) (end 93.81 119.81) (width 0.2) (layer "F.Cu") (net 13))
 (segment (start 100.533722 123.033722) (end 97.31 119.81) (width 0.2) (layer "F.Cu") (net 13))
 (segment (start 100.533722 138.5) (end 100.533722 123.033722) (width 0.2) (layer "F.Cu") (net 13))
 (segment (start 95.5 132) (end 94 132) (width 0.2) (layer "F.Cu") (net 9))
 (segment (start 93.81 112.19) (end 95.19 112.19) (width 0.2) (layer "F.Cu") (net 9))
 (segment (start 96.5 113.5) (end 96.5 118.5) (width 0.2) (layer "F.Cu") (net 9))
 (segment (start 94 132) (end 91.5 132) (width 0.2) (layer "F.Cu") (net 9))
 (segment (start 88.5 132) (end 79.5 132) (width 0.2) (layer "F.Cu") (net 9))
 (segment (start 94 124.5) (end 94 132) (width 0.2) (layer "F.Cu") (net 9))
 (segment (start 96.5 122) (end 94 124.5) (width 0.2) (layer "F.Cu") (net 9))
 (segment (start 88.48 132.02) (end 88.5 132) (width 0.2) (layer "F.Cu") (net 9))
 (segment (start 91.5 132) (end 88.5 132) (width 0.2) (layer "F.Cu") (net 9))
 (segment (start 91.52 132.02) (end 91.5 132) (width 0.2) (layer "F.Cu") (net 9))
 (segment (start 95.19 112.19) (end 96.5 113.5) (width 0.2) (layer "F.Cu") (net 9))
 (segment (start 95.5 132) (end 98.5 135) (width 0.2) (layer "F.Cu") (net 9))
 (segment (start 98.5 138.5) (end 98.5 135) (width 0.2) (layer "F.Cu") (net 9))
 (segment (start 91.52 134.92) (end 91.52 132.02) (width 0.2) (layer "F.Cu") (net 9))
 (segment (start 74.5 132) (end 74.5 138.4) (width 0.2) (layer "F.Cu") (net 9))
 (segment (start 88.48 134.92) (end 88.48 132.02) (width 0.2) (layer "F.Cu") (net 9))
 (via (at 74.5 132) (size 0.6) (drill 0.3) (layers "F.Cu" "B.Cu") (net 9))
 (via (at 96.5 122) (size 0.6) (drill 0.3) (layers "F.Cu" "B.Cu") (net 9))
 (via (at 96.5 118.5) (size 0.6) (drill 0.3) (layers "F.Cu" "B.Cu") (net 9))
 (via (at 79.5 132) (size 0.6) (drill 0.3) (layers "F.Cu" "B.Cu") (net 9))
 (segment (start 96.5 118.5) (end 96.5 122) (width 0.2) (layer "B.Cu") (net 9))
 (segment (start 79.5 132) (end 74.5 132) (width 0.2) (layer "B.Cu") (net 9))
 (segment (start 82.23 117.27) (end 86.19 117.27) (width 0.2) (layer "F.Cu") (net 8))
 (segment (start 76.5 123) (end 82.23 117.27) (width 0.2) (layer "F.Cu") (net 8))
 (segment (start 76.5 138.4) (end 76.5 123) (width 0.2) (layer "F.Cu") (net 8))
 (segment (start 90.5 134.92) (end 90.5 133) (width 0.2) (layer "F.Cu") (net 3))
 (via (at 90.5 133) (size 0.6) (drill 0.3) (layers "F.Cu" "B.Cu") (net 3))
 (segment (start 90.5 133) (end 88 130.5) (width 0.2) (layer "B.Cu") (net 3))
 (segment (start 95.81 128.5) (end 97.31 130) (width 0.2) (layer "B.Cu") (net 3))
 (segment (start 88 129) (end 88.5 128.5) (width 0.2) (layer "B.Cu") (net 3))
 (segment (start 88.5 128.5) (end 95.81 128.5) (width 0.2) (layer "B.Cu") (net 3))
 (segment (start 88 130.5) (end 88 129) (width 0.2) (layer "B.Cu") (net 3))
 (segment (start 89.5 134.92) (end 89.5 133) (width 0.2) (layer "F.Cu") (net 1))
 (via (at 89.5 133) (size 0.6) (drill 0.3) (layers "F.Cu" "B.Cu") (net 1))
 (segment (start 89.5 133) (end 87 133) (width 0.2) (layer "B.Cu") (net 1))
 (segment (start 82.19 128.19) (end 82.19 126.5) (width 0.2) (layer "B.Cu") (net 1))
 (segment (start 87 133) (end 82.19 128.19) (width 0.2) (layer "B.Cu") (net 1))
 (segment (start 92.08 113) (end 92 113) (width 0.2) (layer "F.Cu") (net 10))
 (segment (start 92 113) (end 92 94.81) (width 0.2) (layer "F.Cu") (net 10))
 (segment (start 92 94.81) (end 95 91.81) (width 0.2) (layer "F.Cu") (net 10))
 (segment (start 93.81 114.73) (end 92.08 113) (width 0.2) (layer "F.Cu") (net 10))
 (segment (start 90.5 97.31) (end 90.5 113.96) (width 0.2) (layer "F.Cu") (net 5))
 (segment (start 85 91.81) (end 90.5 97.31) (width 0.2) (layer "F.Cu") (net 5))
 (segment (start 90.5 113.96) (end 93.81 117.27) (width 0.2) (layer "F.Cu") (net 5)))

